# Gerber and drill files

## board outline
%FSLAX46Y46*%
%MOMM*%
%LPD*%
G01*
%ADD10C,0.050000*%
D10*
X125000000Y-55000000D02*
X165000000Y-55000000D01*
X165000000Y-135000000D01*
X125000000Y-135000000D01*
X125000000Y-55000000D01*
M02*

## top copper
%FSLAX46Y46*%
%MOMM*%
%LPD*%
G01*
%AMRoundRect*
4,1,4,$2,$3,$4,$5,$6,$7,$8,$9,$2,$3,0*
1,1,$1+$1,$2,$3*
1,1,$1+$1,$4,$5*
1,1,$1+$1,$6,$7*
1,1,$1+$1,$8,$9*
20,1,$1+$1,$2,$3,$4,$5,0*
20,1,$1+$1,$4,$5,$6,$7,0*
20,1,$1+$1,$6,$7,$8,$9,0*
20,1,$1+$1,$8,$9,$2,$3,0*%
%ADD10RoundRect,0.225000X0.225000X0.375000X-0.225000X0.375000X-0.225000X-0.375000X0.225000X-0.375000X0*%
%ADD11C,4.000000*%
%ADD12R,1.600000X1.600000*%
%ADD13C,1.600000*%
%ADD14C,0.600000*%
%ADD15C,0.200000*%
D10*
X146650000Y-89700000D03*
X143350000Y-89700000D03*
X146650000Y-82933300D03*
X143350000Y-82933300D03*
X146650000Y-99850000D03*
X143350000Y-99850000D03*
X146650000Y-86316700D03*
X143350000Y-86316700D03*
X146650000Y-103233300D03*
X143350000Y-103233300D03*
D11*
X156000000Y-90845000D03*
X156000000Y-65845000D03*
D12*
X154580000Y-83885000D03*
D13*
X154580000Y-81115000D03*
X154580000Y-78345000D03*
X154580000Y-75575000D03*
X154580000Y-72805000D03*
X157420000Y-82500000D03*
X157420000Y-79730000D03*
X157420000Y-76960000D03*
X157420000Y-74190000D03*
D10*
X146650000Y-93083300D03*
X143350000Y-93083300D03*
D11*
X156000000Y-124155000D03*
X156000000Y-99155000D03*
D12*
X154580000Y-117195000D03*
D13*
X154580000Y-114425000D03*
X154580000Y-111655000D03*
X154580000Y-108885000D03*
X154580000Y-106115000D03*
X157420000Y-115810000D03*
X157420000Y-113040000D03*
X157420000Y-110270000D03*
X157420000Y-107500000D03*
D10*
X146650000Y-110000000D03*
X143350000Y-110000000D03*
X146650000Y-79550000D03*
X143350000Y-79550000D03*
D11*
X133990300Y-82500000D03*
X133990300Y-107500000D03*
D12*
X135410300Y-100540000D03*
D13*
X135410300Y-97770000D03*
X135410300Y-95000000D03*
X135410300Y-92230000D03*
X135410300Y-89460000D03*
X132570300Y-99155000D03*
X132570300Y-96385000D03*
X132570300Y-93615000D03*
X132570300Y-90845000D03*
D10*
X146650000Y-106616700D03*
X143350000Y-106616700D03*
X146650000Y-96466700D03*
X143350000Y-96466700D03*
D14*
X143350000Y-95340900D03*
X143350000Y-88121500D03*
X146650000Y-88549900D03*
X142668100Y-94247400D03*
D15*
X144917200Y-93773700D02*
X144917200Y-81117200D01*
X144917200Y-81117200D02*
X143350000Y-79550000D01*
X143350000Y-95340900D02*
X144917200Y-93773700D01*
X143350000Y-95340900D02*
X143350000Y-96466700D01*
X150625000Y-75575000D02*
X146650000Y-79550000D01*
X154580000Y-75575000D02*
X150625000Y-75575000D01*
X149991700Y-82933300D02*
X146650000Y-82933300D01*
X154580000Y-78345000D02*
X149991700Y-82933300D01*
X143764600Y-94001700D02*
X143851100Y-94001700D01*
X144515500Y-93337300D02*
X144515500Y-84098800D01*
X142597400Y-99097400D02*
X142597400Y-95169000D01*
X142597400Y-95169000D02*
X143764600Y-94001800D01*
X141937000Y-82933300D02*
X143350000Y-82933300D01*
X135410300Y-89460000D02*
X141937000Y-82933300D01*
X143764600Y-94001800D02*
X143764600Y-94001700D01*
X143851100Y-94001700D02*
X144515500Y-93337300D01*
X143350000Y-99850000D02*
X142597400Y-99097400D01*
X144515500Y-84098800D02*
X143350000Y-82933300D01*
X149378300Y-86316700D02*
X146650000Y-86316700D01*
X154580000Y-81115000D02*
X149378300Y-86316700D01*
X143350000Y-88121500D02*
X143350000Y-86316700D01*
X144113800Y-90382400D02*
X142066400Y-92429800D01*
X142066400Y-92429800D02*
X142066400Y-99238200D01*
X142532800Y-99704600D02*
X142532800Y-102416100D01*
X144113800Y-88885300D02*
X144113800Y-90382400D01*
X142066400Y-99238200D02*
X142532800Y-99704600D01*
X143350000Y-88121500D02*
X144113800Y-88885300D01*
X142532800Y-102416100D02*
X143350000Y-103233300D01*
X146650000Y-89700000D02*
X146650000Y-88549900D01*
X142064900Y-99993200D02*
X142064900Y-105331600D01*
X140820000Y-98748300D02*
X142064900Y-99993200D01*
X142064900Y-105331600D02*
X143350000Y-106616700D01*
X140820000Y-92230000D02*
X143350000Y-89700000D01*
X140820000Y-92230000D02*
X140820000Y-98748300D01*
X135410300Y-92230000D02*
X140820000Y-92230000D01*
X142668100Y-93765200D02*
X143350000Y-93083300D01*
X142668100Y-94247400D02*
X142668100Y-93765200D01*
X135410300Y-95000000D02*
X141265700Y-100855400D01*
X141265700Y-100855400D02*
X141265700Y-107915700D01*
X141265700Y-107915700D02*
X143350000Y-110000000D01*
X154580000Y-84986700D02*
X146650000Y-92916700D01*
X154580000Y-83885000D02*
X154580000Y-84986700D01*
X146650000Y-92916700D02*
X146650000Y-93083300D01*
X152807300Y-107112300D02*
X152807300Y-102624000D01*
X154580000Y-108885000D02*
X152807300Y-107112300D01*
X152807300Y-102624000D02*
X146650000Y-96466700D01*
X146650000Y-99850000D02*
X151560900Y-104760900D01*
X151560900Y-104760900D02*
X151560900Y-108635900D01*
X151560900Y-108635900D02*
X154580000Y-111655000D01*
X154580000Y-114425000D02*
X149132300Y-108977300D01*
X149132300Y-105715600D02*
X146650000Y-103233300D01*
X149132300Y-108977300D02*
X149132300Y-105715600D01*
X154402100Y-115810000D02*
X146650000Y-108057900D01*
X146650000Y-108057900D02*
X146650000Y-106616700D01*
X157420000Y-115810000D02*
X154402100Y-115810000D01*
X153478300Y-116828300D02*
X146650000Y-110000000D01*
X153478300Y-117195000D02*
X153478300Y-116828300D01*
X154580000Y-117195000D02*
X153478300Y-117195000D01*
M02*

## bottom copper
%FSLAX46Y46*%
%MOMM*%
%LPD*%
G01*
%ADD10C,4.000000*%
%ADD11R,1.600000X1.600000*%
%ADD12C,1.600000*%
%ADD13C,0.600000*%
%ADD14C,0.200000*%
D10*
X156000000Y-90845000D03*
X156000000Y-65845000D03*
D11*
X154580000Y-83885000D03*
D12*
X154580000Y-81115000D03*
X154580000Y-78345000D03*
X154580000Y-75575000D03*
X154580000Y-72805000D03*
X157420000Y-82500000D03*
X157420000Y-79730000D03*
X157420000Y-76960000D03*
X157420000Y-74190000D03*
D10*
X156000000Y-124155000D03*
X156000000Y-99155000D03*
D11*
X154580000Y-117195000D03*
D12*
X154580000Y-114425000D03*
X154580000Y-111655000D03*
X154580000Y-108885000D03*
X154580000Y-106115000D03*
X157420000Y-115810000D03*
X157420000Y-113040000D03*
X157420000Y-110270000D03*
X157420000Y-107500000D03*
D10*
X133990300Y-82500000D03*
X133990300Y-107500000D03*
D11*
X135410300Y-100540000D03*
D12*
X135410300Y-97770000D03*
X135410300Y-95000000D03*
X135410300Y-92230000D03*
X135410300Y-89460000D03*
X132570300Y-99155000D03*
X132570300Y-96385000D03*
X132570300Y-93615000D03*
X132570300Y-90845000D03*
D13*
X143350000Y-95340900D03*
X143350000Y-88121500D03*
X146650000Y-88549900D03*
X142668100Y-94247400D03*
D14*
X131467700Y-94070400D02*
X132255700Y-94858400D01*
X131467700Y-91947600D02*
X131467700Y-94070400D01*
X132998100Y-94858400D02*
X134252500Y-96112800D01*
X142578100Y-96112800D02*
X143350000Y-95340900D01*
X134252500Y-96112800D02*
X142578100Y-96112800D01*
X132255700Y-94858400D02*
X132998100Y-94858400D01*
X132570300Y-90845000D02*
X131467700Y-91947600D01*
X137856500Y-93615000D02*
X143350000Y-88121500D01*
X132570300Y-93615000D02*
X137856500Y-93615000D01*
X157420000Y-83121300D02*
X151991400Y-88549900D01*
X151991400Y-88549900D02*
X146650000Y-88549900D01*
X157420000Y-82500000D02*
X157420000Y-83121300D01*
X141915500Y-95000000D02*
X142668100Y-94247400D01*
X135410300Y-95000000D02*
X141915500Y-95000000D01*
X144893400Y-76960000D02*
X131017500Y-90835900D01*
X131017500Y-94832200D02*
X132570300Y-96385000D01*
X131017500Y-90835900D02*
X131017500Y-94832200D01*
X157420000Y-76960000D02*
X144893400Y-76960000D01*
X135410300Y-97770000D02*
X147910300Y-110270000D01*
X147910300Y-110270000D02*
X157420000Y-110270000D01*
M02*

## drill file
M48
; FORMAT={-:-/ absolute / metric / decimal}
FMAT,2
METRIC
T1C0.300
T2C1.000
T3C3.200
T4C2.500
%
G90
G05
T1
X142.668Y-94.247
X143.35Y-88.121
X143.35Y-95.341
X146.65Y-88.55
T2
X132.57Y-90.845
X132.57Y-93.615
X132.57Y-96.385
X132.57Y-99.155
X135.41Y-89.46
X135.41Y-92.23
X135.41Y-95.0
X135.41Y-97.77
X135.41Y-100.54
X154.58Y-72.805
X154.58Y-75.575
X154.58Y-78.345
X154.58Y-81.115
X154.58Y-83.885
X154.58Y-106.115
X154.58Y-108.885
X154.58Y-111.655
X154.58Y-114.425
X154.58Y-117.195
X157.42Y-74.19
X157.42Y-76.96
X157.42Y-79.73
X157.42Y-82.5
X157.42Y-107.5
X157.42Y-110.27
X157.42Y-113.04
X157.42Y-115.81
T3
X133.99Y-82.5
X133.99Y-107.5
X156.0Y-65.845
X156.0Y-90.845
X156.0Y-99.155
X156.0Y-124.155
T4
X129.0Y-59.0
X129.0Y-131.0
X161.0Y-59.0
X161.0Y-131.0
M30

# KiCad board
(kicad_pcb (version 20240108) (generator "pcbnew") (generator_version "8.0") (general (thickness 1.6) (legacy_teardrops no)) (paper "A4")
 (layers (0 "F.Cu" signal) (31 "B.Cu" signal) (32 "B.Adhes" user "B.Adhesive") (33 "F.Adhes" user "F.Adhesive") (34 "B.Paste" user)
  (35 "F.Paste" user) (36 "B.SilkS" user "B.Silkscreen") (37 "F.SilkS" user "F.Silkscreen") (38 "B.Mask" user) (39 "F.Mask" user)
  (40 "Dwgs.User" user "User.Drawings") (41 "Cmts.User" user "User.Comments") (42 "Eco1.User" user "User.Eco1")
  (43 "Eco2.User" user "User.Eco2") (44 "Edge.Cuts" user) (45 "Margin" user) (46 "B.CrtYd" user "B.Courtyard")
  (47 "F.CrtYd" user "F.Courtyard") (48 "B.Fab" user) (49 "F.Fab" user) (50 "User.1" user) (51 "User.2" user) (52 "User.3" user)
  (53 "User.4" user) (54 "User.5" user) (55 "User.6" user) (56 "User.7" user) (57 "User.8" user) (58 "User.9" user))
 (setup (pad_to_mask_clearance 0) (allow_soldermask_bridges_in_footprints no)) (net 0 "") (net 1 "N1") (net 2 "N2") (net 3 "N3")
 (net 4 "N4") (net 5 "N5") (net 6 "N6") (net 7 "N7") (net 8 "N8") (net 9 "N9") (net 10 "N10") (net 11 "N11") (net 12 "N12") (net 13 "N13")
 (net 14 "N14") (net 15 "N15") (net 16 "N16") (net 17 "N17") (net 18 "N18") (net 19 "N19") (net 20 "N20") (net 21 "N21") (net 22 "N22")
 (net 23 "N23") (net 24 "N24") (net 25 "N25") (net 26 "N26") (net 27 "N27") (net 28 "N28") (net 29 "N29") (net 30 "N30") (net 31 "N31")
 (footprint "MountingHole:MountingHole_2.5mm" (layer "F.Cu") (at 129 131)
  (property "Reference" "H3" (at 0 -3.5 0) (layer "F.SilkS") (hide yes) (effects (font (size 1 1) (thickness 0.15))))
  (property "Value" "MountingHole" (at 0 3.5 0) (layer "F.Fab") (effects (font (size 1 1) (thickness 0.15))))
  (pad "" np_thru_hole circle (at 0 0) (size 2.5 2.5) (drill 2.5) (layers "*.Cu" "*.Mask")))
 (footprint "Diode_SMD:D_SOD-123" (layer "F.Cu") (at 145 89.7 180)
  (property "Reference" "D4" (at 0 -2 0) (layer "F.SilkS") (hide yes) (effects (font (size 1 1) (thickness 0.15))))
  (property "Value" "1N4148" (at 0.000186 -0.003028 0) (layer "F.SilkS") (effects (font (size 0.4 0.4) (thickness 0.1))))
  (pad "1" smd roundrect (at -1.65 0 180) (size 0.9 1.2) (layers "F.Cu" "F.Paste" "F.Mask") (roundrect_rratio 0.25) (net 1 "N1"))
  (pad "2" smd roundrect (at 1.65 0 180) (size 0.9 1.2) (layers "F.Cu" "F.Paste" "F.Mask") (roundrect_rratio 0.25) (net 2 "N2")))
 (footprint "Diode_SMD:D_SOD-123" (layer "F.Cu") (at 145 82.9333 180)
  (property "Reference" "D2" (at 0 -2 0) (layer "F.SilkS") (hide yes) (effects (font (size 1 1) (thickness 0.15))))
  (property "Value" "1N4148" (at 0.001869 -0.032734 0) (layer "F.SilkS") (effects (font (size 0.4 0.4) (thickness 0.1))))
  (pad "1" smd roundrect (at -1.65 0 180) (size 0.9 1.2) (layers "F.Cu" "F.Paste" "F.Mask") (roundrect_rratio 0.25) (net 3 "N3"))
  (pad "2" smd roundrect (at 1.65 0 180) (size 0.9 1.2) (layers "F.Cu" "F.Paste" "F.Mask") (roundrect_rratio 0.25) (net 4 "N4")))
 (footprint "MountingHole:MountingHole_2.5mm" (layer "F.Cu") (at 161 59)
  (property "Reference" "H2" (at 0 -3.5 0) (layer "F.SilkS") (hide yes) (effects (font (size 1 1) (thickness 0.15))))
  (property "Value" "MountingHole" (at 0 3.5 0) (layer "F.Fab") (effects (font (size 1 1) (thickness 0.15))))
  (pad "" np_thru_hole circle (at 0 0) (size 2.5 2.5) (drill 2.5) (layers "*.Cu" "*.Mask")))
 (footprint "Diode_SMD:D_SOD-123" (layer "F.Cu") (at 145 99.85 180)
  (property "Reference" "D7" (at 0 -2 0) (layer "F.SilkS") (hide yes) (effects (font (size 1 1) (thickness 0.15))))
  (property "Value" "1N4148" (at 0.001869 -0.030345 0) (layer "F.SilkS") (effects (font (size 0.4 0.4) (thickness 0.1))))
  (pad "1" smd roundrect (at -1.65 0 180) (size 0.9 1.2) (layers "F.Cu" "F.Paste" "F.Mask") (roundrect_rratio 0.25) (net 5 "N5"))
  (pad "2" smd roundrect (at 1.65 0 180) (size 0.9 1.2) (layers "F.Cu" "F.Paste" "F.Mask") (roundrect_rratio 0.25) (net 4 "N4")))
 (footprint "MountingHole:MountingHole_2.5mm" (layer "F.Cu") (at 129 59)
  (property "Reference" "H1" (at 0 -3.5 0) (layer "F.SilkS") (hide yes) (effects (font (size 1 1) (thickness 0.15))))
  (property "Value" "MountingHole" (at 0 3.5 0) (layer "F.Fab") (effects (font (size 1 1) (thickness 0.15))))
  (pad "" np_thru_hole circle (at 0 0) (size 2.5 2.5) (drill 2.5) (layers "*.Cu" "*.Mask")))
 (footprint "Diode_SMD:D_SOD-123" (layer "F.Cu") (at 145 86.3167 180)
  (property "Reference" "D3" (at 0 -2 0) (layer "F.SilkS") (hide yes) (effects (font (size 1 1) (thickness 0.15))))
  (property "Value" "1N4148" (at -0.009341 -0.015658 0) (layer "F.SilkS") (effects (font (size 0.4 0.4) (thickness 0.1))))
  (pad "1" smd roundrect (at -1.65 0 180) (size 0.9 1.2) (layers "F.Cu" "F.Paste" "F.Mask") (roundrect_rratio 0.25) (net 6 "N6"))
  (pad "2" smd roundrect (at 1.65 0 180) (size 0.9 1.2) (layers "F.Cu" "F.Paste" "F.Mask") (roundrect_rratio 0.25) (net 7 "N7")))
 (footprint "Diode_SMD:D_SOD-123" (layer "F.Cu") (at 145 103.2333 180)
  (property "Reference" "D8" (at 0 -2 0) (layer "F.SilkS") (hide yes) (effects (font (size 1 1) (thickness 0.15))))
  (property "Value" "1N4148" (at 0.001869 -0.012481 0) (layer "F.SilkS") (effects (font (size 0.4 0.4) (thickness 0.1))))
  (pad "1" smd roundrect (at -1.65 0 180) (size 0.9 1.2) (layers "F.Cu" "F.Paste" "F.Mask") (roundrect_rratio 0.25) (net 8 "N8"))
  (pad "2" smd roundrect (at 1.65 0 180) (size 0.9 1.2) (layers "F.Cu" "F.Paste" "F.Mask") (roundrect_rratio 0.25) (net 7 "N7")))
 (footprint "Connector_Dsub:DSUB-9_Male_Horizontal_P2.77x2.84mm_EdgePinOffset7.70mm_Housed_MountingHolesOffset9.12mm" (layer "F.Cu")
  (at 154.58 83.885 90)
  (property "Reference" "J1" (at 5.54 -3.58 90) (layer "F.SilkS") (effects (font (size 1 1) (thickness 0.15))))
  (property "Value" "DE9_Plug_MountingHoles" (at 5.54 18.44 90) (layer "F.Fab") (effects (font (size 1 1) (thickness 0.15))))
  (pad "0" thru_hole circle (at -6.96 1.42 90) (size 4 4) (drill 3.2) (layers "*.Cu" "*.Mask") (remove_unused_layers no) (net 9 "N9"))
  (pad "0" thru_hole circle (at 18.04 1.42 90) (size 4 4) (drill 3.2) (layers "*.Cu" "*.Mask") (remove_unused_layers no) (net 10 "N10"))
  (pad "1" thru_hole rect (at 0 0 90) (size 1.6 1.6) (drill 1) (layers "*.Cu" "*.Mask") (remove_unused_layers no) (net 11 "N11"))
  (pad "2" thru_hole circle (at 2.77 0 90) (size 1.6 1.6) (drill 1) (layers "*.Cu" "*.Mask") (remove_unused_layers no) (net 6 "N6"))
  (pad "3" thru_hole circle (at 5.54 0 90) (size 1.6 1.6) (drill 1) (layers "*.Cu" "*.Mask") (remove_unused_layers no) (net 3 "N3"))
  (pad "4" thru_hole circle (at 8.31 0 90) (size 1.6 1.6) (drill 1) (layers "*.Cu" "*.Mask") (remove_unused_layers no) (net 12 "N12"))
  (pad "5" thru_hole circle (at 11.08 0 90) (size 1.6 1.6) (drill 1) (layers "*.Cu" "*.Mask") (remove_unused_layers no) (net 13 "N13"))
  (pad "6" thru_hole circle (at 1.385 2.84 90) (size 1.6 1.6) (drill 1) (layers "*.Cu" "*.Mask") (remove_unused_layers no) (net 1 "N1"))
  (pad "7" thru_hole circle (at 4.155 2.84 90) (size 1.6 1.6) (drill 1) (layers "*.Cu" "*.Mask") (remove_unused_layers no) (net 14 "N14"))
  (pad "8" thru_hole circle (at 6.925 2.84 90) (size 1.6 1.6) (drill 1) (layers "*.Cu" "*.Mask") (remove_unused_layers no) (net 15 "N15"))
  (pad "9" thru_hole circle (at 9.695 2.84 90) (size 1.6 1.6) (drill 1) (layers "*.Cu" "*.Mask") (remove_unused_layers no) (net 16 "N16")))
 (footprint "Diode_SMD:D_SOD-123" (layer "F.Cu") (at 145 93.0833 180)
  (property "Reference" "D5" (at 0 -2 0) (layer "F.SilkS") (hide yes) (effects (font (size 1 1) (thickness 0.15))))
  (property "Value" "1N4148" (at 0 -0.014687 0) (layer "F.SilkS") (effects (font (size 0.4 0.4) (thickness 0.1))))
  (pad "1" smd roundrect (at -1.65 0 180) (size 0.9 1.2) (layers "F.Cu" "F.Paste" "F.Mask") (roundrect_rratio 0.25) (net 11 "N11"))
  (pad "2" smd roundrect (at 1.65 0 180) (size 0.9 1.2) (layers "F.Cu" "F.Paste" "F.Mask") (roundrect_rratio 0.25) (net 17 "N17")))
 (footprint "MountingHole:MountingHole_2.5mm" (layer "F.Cu") (at 161 131)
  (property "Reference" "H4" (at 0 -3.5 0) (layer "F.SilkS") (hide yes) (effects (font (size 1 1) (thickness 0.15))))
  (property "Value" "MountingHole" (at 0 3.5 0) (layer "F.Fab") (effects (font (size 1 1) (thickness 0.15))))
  (pad "" np_thru_hole circle (at 0 0) (size 2.5 2.5) (drill 2.5) (layers "*.Cu" "*.Mask")))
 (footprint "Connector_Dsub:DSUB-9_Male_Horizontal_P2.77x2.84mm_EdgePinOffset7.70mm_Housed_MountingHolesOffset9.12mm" (layer "F.Cu")
  (at 154.58 117.195 90)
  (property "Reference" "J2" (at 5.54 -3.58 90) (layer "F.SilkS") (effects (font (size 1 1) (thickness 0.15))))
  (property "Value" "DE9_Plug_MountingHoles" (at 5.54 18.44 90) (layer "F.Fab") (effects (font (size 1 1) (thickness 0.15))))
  (pad "0" thru_hole circle (at -6.96 1.42 90) (size 4 4) (drill 3.2) (layers "*.Cu" "*.Mask") (remove_unused_layers no) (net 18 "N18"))
  (pad "0" thru_hole circle (at 18.04 1.42 90) (size 4 4) (drill 3.2) (layers "*.Cu" "*.Mask") (remove_unused_layers no) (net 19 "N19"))
  (pad "1" thru_hole rect (at 0 0 90) (size 1.6 1.6) (drill 1) (layers "*.Cu" "*.Mask") (remove_unused_layers no) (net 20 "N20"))
  (pad "2" thru_hole circle (at 2.77 0 90) (size 1.6 1.6) (drill 1) (layers "*.Cu" "*.Mask") (remove_unused_layers no) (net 8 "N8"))
  (pad "3" thru_hole circle (at 5.54 0 90) (size 1.6 1.6) (drill 1) (layers "*.Cu" "*.Mask") (remove_unused_layers no) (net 5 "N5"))
  (pad "4" thru_hole circle (at 8.31 0 90) (size 1.6 1.6) (drill 1) (layers "*.Cu" "*.Mask") (remove_unused_layers no) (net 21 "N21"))
  (pad "5" thru_hole circle (at 11.08 0 90) (size 1.6 1.6) (drill 1) (layers "*.Cu" "*.Mask") (remove_unused_layers no) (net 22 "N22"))
  (pad "6" thru_hole circle (at 1.385 2.84 90) (size 1.6 1.6) (drill 1) (layers "*.Cu" "*.Mask") (remove_unused_layers no) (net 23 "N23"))
  (pad "7" thru_hole circle (at 4.155 2.84 90) (size 1.6 1.6) (drill 1) (layers "*.Cu" "*.Mask") (remove_unused_layers no) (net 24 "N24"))
  (pad "8" thru_hole circle (at 6.925 2.84 90) (size 1.6 1.6) (drill 1) (layers "*.Cu" "*.Mask") (remove_unused_layers no) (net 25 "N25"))
  (pad "9" thru_hole circle (at 9.695 2.84 90) (size 1.6 1.6) (drill 1) (layers "*.Cu" "*.Mask") (remove_unused_layers no) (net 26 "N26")))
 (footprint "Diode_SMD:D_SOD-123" (layer "F.Cu") (at 145 110 180)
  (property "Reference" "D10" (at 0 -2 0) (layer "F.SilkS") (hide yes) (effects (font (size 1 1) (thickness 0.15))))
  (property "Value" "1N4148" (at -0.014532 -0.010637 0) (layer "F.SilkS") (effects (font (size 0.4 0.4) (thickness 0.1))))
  (pad "1" smd roundrect (at -1.65 0 180) (size 0.9 1.2) (layers "F.Cu" "F.Paste" "F.Mask") (roundrect_rratio 0.25) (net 20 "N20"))
  (pad "2" smd roundrect (at 1.65 0 180) (size 0.9 1.2) (layers "F.Cu" "F.Paste" "F.Mask") (roundrect_rratio 0.25) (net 17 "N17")))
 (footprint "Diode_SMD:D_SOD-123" (layer "F.Cu") (at 145 79.55 180)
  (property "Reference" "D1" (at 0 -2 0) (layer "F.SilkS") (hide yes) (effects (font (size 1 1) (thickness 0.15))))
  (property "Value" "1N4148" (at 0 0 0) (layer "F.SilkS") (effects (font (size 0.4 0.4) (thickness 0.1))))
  (pad "1" smd roundrect (at -1.65 0 180) (size 0.9 1.2) (layers "F.Cu" "F.Paste" "F.Mask") (roundrect_rratio 0.25) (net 12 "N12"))
  (pad "2" smd roundrect (at 1.65 0 180) (size 0.9 1.2) (layers "F.Cu" "F.Paste" "F.Mask") (roundrect_rratio 0.25) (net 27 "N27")))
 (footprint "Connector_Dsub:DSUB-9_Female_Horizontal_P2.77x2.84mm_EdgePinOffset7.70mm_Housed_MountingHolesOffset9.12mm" (layer "F.Cu")
  (at 135.4103 100.54 -90)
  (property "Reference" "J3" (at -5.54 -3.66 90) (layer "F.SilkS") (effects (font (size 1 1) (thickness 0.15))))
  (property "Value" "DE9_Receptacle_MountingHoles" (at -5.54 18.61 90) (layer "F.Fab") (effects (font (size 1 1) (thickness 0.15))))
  (pad "0" thru_hole circle (at -18.04 1.42 270) (size 4 4) (drill 3.2) (layers "*.Cu" "*.Mask") (remove_unused_layers no) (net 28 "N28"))
  (pad "0" thru_hole circle (at 6.96 1.42 270) (size 4 4) (drill 3.2) (layers "*.Cu" "*.Mask") (remove_unused_layers no) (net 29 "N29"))
  (pad "1" thru_hole rect (at 0 0 270) (size 1.6 1.6) (drill 1) (layers "*.Cu" "*.Mask") (remove_unused_layers no) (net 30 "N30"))
  (pad "2" thru_hole circle (at -2.77 0 270) (size 1.6 1.6) (drill 1) (layers "*.Cu" "*.Mask") (remove_unused_layers no) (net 25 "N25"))
  (pad "3" thru_hole circle (at -5.54 0 270) (size 1.6 1.6) (drill 1) (layers "*.Cu" "*.Mask") (remove_unused_layers no) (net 17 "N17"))
  (pad "4" thru_hole circle (at -8.31 0 270) (size 1.6 1.6) (drill 1) (layers "*.Cu" "*.Mask") (remove_unused_layers no) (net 2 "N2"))
  (pad "5" thru_hole circle (at -11.08 0 270) (size 1.6 1.6) (drill 1) (layers "*.Cu" "*.Mask") (remove_unused_layers no) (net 4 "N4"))
  (pad "6" thru_hole circle (at -1.385 2.84 270) (size 1.6 1.6) (drill 1) (layers "*.Cu" "*.Mask") (remove_unused_layers no) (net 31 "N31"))
  (pad "7" thru_hole circle (at -4.155 2.84 270) (size 1.6 1.6) (drill 1) (layers "*.Cu" "*.Mask") (remove_unused_layers no) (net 15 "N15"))
  (pad "8" thru_hole circle (at -6.925 2.84 270) (size 1.6 1.6) (drill 1) (layers "*.Cu" "*.Mask") (remove_unused_layers no) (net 7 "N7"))
  (pad "9" thru_hole circle (at -9.695 2.84 270) (size 1.6 1.6) (drill 1) (layers "*.Cu" "*.Mask") (remove_unused_layers no) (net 27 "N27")))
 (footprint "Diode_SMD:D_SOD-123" (layer "F.Cu") (at 145 106.6167 180)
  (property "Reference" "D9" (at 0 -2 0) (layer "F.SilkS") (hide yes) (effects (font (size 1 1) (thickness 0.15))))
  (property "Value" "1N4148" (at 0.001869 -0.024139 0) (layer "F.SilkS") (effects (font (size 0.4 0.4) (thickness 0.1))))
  (pad "1" smd roundrect (at -1.65 0 180) (size 0.9 1.2) (layers "F.Cu" "F.Paste" "F.Mask") (roundrect_rratio 0.25) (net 23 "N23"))
  (pad "2" smd roundrect (at 1.65 0 180) (size 0.9 1.2) (layers "F.Cu" "F.Paste" "F.Mask") (roundrect_rratio 0.25) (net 2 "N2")))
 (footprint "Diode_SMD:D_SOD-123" (layer "F.Cu") (at 145 96.4667 180)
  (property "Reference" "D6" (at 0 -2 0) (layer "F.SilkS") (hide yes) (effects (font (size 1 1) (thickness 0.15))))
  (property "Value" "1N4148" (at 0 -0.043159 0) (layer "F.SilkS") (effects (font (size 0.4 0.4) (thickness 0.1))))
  (pad "1" smd roundrect (at -1.65 0 180) (size 0.9 1.2) (layers "F.Cu" "F.Paste" "F.Mask") (roundrect_rratio 0.25) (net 21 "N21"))
  (pad "2" smd roundrect (at 1.65 0 180) (size 0.9 1.2) (layers "F.Cu" "F.Paste" "F.Mask") (roundrect_rratio 0.25) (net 27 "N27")))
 (gr_rect (start 125 55) (end 165 135) (stroke (width 0.05) (type default)) (fill none) (layer "Edge.Cuts"))
 (segment (start 144.9172 93.7737) (end 144.9172 81.1172) (width 0.2) (layer "F.Cu") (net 27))
 (segment (start 144.9172 81.1172) (end 143.35 79.55) (width 0.2) (layer "F.Cu") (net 27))
 (segment (start 143.35 95.3409) (end 144.9172 93.7737) (width 0.2) (layer "F.Cu") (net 27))
 (segment (start 143.35 95.3409) (end 143.35 96.4667) (width 0.2) (layer "F.Cu") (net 27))
 (via (at 143.35 95.3409) (size 0.6) (drill 0.3) (layers "F.Cu" "B.Cu") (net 27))
 (segment (start 131.4677 94.0704) (end 132.2557 94.8584) (width 0.2) (layer "B.Cu") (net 27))
 (segment (start 131.4677 91.9476) (end 131.4677 94.0704) (width 0.2) (layer "B.Cu") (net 27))
 (segment (start 132.9981 94.8584) (end 134.2525 96.1128) (width 0.2) (layer "B.Cu") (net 27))
 (segment (start 142.5781 96.1128) (end 143.35 95.3409) (width 0.2) (layer "B.Cu") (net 27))
 (segment (start 134.2525 96.1128) (end 142.5781 96.1128) (width 0.2) (layer "B.Cu") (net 27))
 (segment (start 132.2557 94.8584) (end 132.9981 94.8584) (width 0.2) (layer "B.Cu") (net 27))
 (segment (start 132.5703 90.845) (end 131.4677 91.9476) (width 0.2) (layer "B.Cu") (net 27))
 (segment (start 150.625 75.575) (end 146.65 79.55) (width 0.2) (layer "F.Cu") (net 12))
 (segment (start 154.58 75.575) (end 150.625 75.575) (width 0.2) (layer "F.Cu") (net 12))
 (segment (start 149.9917 82.9333) (end 146.65 82.9333) (width 0.2) (layer "F.Cu") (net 3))
 (segment (start 154.58 78.345) (end 149.9917 82.9333) (width 0.2) (layer "F.Cu") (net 3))
 (segment (start 143.7646 94.0017) (end 143.8511 94.0017) (width 0.2) (layer "F.Cu") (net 4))
 (segment (start 144.5155 93.3373) (end 144.5155 84.0988) (width 0.2) (layer "F.Cu") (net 4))
 (segment (start 142.5974 99.0974) (end 142.5974 95.169) (width 0.2) (layer "F.Cu") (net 4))
 (segment (start 142.5974 95.169) (end 143.7646 94.0018) (width 0.2) (layer "F.Cu") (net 4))
 (segment (start 141.937 82.9333) (end 143.35 82.9333) (width 0.2) (layer "F.Cu") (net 4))
 (segment (start 135.4103 89.46) (end 141.937 82.9333) (width 0.2) (layer "F.Cu") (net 4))
 (segment (start 143.7646 94.0018) (end 143.7646 94.0017) (width 0.2) (layer "F.Cu") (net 4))
 (segment (start 143.8511 94.0017) (end 144.5155 93.3373) (width 0.2) (layer "F.Cu") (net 4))
 (segment (start 143.35 99.85) (end 142.5974 99.0974) (width 0.2) (layer "F.Cu") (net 4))
 (segment (start 144.5155 84.0988) (end 143.35 82.9333) (width 0.2) (layer "F.Cu") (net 4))
 (segment (start 149.3783 86.3167) (end 146.65 86.3167) (width 0.2) (layer "F.Cu") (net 6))
 (segment (start 154.58 81.115) (end 149.3783 86.3167) (width 0.2) (layer "F.Cu") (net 6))
 (segment (start 143.35 88.1215) (end 143.35 86.3167) (width 0.2) (layer "F.Cu") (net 7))
 (segment (start 144.1138 90.3824) (end 142.0664 92.4298) (width 0.2) (layer "F.Cu") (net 7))
 (segment (start 142.0664 92.4298) (end 142.0664 99.2382) (width 0.2) (layer "F.Cu") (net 7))
 (segment (start 142.5328 99.7046) (end 142.5328 102.4161) (width 0.2) (layer "F.Cu") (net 7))
 (segment (start 144.1138 88.8853) (end 144.1138 90.3824) (width 0.2) (layer "F.Cu") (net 7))
 (segment (start 142.0664 99.2382) (end 142.5328 99.7046) (width 0.2) (layer "F.Cu") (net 7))
 (segment (start 143.35 88.1215) (end 144.1138 88.8853) (width 0.2) (layer "F.Cu") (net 7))
 (segment (start 142.5328 102.4161) (end 143.35 103.2333) (width 0.2) (layer "F.Cu") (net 7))
 (via (at 143.35 88.1215) (size 0.6) (drill 0.3) (layers "F.Cu" "B.Cu") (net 7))
 (segment (start 137.8565 93.615) (end 143.35 88.1215) (width 0.2) (layer "B.Cu") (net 7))
 (segment (start 132.5703 93.615) (end 137.8565 93.615) (width 0.2) (layer "B.Cu") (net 7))
 (segment (start 146.65 89.7) (end 146.65 88.5499) (width 0.2) (layer "F.Cu") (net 1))
 (via (at 146.65 88.5499) (size 0.6) (drill 0.3) (layers "F.Cu" "B.Cu") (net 1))
 (segment (start 157.42 83.1213) (end 151.9914 88.5499) (width 0.2) (layer "B.Cu") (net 1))
 (segment (start 151.9914 88.5499) (end 146.65 88.5499) (width 0.2) (layer "B.Cu") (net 1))
 (segment (start 157.42 82.5) (end 157.42 83.1213) (width 0.2) (layer "B.Cu") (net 1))
 (segment (start 142.0649 99.9932) (end 142.0649 105.3316) (width 0.2) (layer "F.Cu") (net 2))
 (segment (start 140.82 98.7483) (end 142.0649 99.9932) (width 0.2) (layer "F.Cu") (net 2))
 (segment (start 142.0649 105.3316) (end 143.35 106.6167) (width 0.2) (layer "F.Cu") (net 2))
 (segment (start 140.82 92.23) (end 143.35 89.7) (width 0.2) (layer "F.Cu") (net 2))
 (segment (start 140.82 92.23) (end 140.82 98.7483) (width 0.2) (layer "F.Cu") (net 2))
 (segment (start 135.4103 92.23) (end 140.82 92.23) (width 0.2) (layer "F.Cu") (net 2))
 (segment (start 142.6681 93.7652) (end 143.35 93.0833) (width 0.2) (layer "F.Cu") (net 17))
 (segment (start 142.6681 94.2474) (end 142.6681 93.7652) (width 0.2) (layer "F.Cu") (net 17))
 (segment (start 135.4103 95) (end 141.2657 100.8554) (width 0.2) (layer "F.Cu") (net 17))
 (segment (start 141.2657 100.8554) (end 141.2657 107.9157) (width 0.2) (layer "F.Cu") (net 17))
 (segment (start 141.2657 107.9157) (end 143.35 110) (width 0.2) (layer "F.Cu") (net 17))
 (via (at 142.6681 94.2474) (size 0.6) (drill 0.3) (layers "F.Cu" "B.Cu") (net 17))
 (segment (start 141.9155 95) (end 142.6681 94.2474) (width 0.2) (layer "B.Cu") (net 17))
 (segment (start 135.4103 95) (end 141.9155 95) (width 0.2) (layer "B.Cu") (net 17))
 (segment (start 154.58 84.9867) (end 146.65 92.9167) (width 0.2) (layer "F.Cu") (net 11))
 (segment (start 154.58 83.885) (end 154.58 84.9867) (width 0.2) (layer "F.Cu") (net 11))
 (segment (start 146.65 92.9167) (end 146.65 93.0833) (width 0.2) (layer "F.Cu") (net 11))
 (segment (start 152.8073 107.1123) (end 152.8073 102.624) (width 0.2) (layer "F.Cu") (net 21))
 (segment (start 154.58 108.885) (end 152.8073 107.1123) (width 0.2) (layer "F.Cu") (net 21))
 (segment (start 152.8073 102.624) (end 146.65 96.4667) (width 0.2) (layer "F.Cu") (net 21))
 (segment (start 146.65 99.85) (end 151.5609 104.7609) (width 0.2) (layer "F.Cu") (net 5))
 (segment (start 151.5609 104.7609) (end 151.5609 108.6359) (width 0.2) (layer "F.Cu") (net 5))
 (segment (start 151.5609 108.6359) (end 154.58 111.655) (width 0.2) (layer "F.Cu") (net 5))
 (segment (start 154.58 114.425) (end 149.1323 108.9773) (width 0.2) (layer "F.Cu") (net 8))
 (segment (start 149.1323 105.7156) (end 146.65 103.2333) (width 0.2) (layer "F.Cu") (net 8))
 (segment (start 149.1323 108.9773) (end 149.1323 105.7156) (width 0.2) (layer "F.Cu") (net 8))
 (segment (start 154.4021 115.81) (end 146.65 108.0579) (width 0.2) (layer "F.Cu") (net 23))
 (segment (start 146.65 108.0579) (end 146.65 106.6167) (width 0.2) (layer "F.Cu") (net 23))
 (segment (start 157.42 115.81) (end 154.4021 115.81) (width 0.2) (layer "F.Cu") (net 23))
 (segment (start 153.4783 116.8283) (end 146.65 110) (width 0.2) (layer "F.Cu") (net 20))
 (segment (start 153.4783 117.195) (end 153.4783 116.8283) (width 0.2) (layer "F.Cu") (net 20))
 (segment (start 154.58 117.195) (end 153.4783 117.195) (width 0.2) (layer "F.Cu") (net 20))
 (segment (start 144.8934 76.96) (end 131.0175 90.8359) (width 0.2) (layer "B.Cu") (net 15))
 (segment (start 131.0175 94.8322) (end 132.5703 96.385) (width 0.2) (layer "B.Cu") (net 15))
 (segment (start 131.0175 90.8359) (end 131.0175 94.8322) (width 0.2) (layer "B.Cu") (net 15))
 (segment (start 157.42 76.96) (end 144.8934 76.96) (width 0.2) (layer "B.Cu") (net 15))
 (segment (start 135.4103 97.77) (end 147.9103 110.27) (width 0.2) (layer "B.Cu") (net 25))
 (segment (start 147.9103 110.27) (end 157.42 110.27) (width 0.2) (layer "B.Cu") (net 25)))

